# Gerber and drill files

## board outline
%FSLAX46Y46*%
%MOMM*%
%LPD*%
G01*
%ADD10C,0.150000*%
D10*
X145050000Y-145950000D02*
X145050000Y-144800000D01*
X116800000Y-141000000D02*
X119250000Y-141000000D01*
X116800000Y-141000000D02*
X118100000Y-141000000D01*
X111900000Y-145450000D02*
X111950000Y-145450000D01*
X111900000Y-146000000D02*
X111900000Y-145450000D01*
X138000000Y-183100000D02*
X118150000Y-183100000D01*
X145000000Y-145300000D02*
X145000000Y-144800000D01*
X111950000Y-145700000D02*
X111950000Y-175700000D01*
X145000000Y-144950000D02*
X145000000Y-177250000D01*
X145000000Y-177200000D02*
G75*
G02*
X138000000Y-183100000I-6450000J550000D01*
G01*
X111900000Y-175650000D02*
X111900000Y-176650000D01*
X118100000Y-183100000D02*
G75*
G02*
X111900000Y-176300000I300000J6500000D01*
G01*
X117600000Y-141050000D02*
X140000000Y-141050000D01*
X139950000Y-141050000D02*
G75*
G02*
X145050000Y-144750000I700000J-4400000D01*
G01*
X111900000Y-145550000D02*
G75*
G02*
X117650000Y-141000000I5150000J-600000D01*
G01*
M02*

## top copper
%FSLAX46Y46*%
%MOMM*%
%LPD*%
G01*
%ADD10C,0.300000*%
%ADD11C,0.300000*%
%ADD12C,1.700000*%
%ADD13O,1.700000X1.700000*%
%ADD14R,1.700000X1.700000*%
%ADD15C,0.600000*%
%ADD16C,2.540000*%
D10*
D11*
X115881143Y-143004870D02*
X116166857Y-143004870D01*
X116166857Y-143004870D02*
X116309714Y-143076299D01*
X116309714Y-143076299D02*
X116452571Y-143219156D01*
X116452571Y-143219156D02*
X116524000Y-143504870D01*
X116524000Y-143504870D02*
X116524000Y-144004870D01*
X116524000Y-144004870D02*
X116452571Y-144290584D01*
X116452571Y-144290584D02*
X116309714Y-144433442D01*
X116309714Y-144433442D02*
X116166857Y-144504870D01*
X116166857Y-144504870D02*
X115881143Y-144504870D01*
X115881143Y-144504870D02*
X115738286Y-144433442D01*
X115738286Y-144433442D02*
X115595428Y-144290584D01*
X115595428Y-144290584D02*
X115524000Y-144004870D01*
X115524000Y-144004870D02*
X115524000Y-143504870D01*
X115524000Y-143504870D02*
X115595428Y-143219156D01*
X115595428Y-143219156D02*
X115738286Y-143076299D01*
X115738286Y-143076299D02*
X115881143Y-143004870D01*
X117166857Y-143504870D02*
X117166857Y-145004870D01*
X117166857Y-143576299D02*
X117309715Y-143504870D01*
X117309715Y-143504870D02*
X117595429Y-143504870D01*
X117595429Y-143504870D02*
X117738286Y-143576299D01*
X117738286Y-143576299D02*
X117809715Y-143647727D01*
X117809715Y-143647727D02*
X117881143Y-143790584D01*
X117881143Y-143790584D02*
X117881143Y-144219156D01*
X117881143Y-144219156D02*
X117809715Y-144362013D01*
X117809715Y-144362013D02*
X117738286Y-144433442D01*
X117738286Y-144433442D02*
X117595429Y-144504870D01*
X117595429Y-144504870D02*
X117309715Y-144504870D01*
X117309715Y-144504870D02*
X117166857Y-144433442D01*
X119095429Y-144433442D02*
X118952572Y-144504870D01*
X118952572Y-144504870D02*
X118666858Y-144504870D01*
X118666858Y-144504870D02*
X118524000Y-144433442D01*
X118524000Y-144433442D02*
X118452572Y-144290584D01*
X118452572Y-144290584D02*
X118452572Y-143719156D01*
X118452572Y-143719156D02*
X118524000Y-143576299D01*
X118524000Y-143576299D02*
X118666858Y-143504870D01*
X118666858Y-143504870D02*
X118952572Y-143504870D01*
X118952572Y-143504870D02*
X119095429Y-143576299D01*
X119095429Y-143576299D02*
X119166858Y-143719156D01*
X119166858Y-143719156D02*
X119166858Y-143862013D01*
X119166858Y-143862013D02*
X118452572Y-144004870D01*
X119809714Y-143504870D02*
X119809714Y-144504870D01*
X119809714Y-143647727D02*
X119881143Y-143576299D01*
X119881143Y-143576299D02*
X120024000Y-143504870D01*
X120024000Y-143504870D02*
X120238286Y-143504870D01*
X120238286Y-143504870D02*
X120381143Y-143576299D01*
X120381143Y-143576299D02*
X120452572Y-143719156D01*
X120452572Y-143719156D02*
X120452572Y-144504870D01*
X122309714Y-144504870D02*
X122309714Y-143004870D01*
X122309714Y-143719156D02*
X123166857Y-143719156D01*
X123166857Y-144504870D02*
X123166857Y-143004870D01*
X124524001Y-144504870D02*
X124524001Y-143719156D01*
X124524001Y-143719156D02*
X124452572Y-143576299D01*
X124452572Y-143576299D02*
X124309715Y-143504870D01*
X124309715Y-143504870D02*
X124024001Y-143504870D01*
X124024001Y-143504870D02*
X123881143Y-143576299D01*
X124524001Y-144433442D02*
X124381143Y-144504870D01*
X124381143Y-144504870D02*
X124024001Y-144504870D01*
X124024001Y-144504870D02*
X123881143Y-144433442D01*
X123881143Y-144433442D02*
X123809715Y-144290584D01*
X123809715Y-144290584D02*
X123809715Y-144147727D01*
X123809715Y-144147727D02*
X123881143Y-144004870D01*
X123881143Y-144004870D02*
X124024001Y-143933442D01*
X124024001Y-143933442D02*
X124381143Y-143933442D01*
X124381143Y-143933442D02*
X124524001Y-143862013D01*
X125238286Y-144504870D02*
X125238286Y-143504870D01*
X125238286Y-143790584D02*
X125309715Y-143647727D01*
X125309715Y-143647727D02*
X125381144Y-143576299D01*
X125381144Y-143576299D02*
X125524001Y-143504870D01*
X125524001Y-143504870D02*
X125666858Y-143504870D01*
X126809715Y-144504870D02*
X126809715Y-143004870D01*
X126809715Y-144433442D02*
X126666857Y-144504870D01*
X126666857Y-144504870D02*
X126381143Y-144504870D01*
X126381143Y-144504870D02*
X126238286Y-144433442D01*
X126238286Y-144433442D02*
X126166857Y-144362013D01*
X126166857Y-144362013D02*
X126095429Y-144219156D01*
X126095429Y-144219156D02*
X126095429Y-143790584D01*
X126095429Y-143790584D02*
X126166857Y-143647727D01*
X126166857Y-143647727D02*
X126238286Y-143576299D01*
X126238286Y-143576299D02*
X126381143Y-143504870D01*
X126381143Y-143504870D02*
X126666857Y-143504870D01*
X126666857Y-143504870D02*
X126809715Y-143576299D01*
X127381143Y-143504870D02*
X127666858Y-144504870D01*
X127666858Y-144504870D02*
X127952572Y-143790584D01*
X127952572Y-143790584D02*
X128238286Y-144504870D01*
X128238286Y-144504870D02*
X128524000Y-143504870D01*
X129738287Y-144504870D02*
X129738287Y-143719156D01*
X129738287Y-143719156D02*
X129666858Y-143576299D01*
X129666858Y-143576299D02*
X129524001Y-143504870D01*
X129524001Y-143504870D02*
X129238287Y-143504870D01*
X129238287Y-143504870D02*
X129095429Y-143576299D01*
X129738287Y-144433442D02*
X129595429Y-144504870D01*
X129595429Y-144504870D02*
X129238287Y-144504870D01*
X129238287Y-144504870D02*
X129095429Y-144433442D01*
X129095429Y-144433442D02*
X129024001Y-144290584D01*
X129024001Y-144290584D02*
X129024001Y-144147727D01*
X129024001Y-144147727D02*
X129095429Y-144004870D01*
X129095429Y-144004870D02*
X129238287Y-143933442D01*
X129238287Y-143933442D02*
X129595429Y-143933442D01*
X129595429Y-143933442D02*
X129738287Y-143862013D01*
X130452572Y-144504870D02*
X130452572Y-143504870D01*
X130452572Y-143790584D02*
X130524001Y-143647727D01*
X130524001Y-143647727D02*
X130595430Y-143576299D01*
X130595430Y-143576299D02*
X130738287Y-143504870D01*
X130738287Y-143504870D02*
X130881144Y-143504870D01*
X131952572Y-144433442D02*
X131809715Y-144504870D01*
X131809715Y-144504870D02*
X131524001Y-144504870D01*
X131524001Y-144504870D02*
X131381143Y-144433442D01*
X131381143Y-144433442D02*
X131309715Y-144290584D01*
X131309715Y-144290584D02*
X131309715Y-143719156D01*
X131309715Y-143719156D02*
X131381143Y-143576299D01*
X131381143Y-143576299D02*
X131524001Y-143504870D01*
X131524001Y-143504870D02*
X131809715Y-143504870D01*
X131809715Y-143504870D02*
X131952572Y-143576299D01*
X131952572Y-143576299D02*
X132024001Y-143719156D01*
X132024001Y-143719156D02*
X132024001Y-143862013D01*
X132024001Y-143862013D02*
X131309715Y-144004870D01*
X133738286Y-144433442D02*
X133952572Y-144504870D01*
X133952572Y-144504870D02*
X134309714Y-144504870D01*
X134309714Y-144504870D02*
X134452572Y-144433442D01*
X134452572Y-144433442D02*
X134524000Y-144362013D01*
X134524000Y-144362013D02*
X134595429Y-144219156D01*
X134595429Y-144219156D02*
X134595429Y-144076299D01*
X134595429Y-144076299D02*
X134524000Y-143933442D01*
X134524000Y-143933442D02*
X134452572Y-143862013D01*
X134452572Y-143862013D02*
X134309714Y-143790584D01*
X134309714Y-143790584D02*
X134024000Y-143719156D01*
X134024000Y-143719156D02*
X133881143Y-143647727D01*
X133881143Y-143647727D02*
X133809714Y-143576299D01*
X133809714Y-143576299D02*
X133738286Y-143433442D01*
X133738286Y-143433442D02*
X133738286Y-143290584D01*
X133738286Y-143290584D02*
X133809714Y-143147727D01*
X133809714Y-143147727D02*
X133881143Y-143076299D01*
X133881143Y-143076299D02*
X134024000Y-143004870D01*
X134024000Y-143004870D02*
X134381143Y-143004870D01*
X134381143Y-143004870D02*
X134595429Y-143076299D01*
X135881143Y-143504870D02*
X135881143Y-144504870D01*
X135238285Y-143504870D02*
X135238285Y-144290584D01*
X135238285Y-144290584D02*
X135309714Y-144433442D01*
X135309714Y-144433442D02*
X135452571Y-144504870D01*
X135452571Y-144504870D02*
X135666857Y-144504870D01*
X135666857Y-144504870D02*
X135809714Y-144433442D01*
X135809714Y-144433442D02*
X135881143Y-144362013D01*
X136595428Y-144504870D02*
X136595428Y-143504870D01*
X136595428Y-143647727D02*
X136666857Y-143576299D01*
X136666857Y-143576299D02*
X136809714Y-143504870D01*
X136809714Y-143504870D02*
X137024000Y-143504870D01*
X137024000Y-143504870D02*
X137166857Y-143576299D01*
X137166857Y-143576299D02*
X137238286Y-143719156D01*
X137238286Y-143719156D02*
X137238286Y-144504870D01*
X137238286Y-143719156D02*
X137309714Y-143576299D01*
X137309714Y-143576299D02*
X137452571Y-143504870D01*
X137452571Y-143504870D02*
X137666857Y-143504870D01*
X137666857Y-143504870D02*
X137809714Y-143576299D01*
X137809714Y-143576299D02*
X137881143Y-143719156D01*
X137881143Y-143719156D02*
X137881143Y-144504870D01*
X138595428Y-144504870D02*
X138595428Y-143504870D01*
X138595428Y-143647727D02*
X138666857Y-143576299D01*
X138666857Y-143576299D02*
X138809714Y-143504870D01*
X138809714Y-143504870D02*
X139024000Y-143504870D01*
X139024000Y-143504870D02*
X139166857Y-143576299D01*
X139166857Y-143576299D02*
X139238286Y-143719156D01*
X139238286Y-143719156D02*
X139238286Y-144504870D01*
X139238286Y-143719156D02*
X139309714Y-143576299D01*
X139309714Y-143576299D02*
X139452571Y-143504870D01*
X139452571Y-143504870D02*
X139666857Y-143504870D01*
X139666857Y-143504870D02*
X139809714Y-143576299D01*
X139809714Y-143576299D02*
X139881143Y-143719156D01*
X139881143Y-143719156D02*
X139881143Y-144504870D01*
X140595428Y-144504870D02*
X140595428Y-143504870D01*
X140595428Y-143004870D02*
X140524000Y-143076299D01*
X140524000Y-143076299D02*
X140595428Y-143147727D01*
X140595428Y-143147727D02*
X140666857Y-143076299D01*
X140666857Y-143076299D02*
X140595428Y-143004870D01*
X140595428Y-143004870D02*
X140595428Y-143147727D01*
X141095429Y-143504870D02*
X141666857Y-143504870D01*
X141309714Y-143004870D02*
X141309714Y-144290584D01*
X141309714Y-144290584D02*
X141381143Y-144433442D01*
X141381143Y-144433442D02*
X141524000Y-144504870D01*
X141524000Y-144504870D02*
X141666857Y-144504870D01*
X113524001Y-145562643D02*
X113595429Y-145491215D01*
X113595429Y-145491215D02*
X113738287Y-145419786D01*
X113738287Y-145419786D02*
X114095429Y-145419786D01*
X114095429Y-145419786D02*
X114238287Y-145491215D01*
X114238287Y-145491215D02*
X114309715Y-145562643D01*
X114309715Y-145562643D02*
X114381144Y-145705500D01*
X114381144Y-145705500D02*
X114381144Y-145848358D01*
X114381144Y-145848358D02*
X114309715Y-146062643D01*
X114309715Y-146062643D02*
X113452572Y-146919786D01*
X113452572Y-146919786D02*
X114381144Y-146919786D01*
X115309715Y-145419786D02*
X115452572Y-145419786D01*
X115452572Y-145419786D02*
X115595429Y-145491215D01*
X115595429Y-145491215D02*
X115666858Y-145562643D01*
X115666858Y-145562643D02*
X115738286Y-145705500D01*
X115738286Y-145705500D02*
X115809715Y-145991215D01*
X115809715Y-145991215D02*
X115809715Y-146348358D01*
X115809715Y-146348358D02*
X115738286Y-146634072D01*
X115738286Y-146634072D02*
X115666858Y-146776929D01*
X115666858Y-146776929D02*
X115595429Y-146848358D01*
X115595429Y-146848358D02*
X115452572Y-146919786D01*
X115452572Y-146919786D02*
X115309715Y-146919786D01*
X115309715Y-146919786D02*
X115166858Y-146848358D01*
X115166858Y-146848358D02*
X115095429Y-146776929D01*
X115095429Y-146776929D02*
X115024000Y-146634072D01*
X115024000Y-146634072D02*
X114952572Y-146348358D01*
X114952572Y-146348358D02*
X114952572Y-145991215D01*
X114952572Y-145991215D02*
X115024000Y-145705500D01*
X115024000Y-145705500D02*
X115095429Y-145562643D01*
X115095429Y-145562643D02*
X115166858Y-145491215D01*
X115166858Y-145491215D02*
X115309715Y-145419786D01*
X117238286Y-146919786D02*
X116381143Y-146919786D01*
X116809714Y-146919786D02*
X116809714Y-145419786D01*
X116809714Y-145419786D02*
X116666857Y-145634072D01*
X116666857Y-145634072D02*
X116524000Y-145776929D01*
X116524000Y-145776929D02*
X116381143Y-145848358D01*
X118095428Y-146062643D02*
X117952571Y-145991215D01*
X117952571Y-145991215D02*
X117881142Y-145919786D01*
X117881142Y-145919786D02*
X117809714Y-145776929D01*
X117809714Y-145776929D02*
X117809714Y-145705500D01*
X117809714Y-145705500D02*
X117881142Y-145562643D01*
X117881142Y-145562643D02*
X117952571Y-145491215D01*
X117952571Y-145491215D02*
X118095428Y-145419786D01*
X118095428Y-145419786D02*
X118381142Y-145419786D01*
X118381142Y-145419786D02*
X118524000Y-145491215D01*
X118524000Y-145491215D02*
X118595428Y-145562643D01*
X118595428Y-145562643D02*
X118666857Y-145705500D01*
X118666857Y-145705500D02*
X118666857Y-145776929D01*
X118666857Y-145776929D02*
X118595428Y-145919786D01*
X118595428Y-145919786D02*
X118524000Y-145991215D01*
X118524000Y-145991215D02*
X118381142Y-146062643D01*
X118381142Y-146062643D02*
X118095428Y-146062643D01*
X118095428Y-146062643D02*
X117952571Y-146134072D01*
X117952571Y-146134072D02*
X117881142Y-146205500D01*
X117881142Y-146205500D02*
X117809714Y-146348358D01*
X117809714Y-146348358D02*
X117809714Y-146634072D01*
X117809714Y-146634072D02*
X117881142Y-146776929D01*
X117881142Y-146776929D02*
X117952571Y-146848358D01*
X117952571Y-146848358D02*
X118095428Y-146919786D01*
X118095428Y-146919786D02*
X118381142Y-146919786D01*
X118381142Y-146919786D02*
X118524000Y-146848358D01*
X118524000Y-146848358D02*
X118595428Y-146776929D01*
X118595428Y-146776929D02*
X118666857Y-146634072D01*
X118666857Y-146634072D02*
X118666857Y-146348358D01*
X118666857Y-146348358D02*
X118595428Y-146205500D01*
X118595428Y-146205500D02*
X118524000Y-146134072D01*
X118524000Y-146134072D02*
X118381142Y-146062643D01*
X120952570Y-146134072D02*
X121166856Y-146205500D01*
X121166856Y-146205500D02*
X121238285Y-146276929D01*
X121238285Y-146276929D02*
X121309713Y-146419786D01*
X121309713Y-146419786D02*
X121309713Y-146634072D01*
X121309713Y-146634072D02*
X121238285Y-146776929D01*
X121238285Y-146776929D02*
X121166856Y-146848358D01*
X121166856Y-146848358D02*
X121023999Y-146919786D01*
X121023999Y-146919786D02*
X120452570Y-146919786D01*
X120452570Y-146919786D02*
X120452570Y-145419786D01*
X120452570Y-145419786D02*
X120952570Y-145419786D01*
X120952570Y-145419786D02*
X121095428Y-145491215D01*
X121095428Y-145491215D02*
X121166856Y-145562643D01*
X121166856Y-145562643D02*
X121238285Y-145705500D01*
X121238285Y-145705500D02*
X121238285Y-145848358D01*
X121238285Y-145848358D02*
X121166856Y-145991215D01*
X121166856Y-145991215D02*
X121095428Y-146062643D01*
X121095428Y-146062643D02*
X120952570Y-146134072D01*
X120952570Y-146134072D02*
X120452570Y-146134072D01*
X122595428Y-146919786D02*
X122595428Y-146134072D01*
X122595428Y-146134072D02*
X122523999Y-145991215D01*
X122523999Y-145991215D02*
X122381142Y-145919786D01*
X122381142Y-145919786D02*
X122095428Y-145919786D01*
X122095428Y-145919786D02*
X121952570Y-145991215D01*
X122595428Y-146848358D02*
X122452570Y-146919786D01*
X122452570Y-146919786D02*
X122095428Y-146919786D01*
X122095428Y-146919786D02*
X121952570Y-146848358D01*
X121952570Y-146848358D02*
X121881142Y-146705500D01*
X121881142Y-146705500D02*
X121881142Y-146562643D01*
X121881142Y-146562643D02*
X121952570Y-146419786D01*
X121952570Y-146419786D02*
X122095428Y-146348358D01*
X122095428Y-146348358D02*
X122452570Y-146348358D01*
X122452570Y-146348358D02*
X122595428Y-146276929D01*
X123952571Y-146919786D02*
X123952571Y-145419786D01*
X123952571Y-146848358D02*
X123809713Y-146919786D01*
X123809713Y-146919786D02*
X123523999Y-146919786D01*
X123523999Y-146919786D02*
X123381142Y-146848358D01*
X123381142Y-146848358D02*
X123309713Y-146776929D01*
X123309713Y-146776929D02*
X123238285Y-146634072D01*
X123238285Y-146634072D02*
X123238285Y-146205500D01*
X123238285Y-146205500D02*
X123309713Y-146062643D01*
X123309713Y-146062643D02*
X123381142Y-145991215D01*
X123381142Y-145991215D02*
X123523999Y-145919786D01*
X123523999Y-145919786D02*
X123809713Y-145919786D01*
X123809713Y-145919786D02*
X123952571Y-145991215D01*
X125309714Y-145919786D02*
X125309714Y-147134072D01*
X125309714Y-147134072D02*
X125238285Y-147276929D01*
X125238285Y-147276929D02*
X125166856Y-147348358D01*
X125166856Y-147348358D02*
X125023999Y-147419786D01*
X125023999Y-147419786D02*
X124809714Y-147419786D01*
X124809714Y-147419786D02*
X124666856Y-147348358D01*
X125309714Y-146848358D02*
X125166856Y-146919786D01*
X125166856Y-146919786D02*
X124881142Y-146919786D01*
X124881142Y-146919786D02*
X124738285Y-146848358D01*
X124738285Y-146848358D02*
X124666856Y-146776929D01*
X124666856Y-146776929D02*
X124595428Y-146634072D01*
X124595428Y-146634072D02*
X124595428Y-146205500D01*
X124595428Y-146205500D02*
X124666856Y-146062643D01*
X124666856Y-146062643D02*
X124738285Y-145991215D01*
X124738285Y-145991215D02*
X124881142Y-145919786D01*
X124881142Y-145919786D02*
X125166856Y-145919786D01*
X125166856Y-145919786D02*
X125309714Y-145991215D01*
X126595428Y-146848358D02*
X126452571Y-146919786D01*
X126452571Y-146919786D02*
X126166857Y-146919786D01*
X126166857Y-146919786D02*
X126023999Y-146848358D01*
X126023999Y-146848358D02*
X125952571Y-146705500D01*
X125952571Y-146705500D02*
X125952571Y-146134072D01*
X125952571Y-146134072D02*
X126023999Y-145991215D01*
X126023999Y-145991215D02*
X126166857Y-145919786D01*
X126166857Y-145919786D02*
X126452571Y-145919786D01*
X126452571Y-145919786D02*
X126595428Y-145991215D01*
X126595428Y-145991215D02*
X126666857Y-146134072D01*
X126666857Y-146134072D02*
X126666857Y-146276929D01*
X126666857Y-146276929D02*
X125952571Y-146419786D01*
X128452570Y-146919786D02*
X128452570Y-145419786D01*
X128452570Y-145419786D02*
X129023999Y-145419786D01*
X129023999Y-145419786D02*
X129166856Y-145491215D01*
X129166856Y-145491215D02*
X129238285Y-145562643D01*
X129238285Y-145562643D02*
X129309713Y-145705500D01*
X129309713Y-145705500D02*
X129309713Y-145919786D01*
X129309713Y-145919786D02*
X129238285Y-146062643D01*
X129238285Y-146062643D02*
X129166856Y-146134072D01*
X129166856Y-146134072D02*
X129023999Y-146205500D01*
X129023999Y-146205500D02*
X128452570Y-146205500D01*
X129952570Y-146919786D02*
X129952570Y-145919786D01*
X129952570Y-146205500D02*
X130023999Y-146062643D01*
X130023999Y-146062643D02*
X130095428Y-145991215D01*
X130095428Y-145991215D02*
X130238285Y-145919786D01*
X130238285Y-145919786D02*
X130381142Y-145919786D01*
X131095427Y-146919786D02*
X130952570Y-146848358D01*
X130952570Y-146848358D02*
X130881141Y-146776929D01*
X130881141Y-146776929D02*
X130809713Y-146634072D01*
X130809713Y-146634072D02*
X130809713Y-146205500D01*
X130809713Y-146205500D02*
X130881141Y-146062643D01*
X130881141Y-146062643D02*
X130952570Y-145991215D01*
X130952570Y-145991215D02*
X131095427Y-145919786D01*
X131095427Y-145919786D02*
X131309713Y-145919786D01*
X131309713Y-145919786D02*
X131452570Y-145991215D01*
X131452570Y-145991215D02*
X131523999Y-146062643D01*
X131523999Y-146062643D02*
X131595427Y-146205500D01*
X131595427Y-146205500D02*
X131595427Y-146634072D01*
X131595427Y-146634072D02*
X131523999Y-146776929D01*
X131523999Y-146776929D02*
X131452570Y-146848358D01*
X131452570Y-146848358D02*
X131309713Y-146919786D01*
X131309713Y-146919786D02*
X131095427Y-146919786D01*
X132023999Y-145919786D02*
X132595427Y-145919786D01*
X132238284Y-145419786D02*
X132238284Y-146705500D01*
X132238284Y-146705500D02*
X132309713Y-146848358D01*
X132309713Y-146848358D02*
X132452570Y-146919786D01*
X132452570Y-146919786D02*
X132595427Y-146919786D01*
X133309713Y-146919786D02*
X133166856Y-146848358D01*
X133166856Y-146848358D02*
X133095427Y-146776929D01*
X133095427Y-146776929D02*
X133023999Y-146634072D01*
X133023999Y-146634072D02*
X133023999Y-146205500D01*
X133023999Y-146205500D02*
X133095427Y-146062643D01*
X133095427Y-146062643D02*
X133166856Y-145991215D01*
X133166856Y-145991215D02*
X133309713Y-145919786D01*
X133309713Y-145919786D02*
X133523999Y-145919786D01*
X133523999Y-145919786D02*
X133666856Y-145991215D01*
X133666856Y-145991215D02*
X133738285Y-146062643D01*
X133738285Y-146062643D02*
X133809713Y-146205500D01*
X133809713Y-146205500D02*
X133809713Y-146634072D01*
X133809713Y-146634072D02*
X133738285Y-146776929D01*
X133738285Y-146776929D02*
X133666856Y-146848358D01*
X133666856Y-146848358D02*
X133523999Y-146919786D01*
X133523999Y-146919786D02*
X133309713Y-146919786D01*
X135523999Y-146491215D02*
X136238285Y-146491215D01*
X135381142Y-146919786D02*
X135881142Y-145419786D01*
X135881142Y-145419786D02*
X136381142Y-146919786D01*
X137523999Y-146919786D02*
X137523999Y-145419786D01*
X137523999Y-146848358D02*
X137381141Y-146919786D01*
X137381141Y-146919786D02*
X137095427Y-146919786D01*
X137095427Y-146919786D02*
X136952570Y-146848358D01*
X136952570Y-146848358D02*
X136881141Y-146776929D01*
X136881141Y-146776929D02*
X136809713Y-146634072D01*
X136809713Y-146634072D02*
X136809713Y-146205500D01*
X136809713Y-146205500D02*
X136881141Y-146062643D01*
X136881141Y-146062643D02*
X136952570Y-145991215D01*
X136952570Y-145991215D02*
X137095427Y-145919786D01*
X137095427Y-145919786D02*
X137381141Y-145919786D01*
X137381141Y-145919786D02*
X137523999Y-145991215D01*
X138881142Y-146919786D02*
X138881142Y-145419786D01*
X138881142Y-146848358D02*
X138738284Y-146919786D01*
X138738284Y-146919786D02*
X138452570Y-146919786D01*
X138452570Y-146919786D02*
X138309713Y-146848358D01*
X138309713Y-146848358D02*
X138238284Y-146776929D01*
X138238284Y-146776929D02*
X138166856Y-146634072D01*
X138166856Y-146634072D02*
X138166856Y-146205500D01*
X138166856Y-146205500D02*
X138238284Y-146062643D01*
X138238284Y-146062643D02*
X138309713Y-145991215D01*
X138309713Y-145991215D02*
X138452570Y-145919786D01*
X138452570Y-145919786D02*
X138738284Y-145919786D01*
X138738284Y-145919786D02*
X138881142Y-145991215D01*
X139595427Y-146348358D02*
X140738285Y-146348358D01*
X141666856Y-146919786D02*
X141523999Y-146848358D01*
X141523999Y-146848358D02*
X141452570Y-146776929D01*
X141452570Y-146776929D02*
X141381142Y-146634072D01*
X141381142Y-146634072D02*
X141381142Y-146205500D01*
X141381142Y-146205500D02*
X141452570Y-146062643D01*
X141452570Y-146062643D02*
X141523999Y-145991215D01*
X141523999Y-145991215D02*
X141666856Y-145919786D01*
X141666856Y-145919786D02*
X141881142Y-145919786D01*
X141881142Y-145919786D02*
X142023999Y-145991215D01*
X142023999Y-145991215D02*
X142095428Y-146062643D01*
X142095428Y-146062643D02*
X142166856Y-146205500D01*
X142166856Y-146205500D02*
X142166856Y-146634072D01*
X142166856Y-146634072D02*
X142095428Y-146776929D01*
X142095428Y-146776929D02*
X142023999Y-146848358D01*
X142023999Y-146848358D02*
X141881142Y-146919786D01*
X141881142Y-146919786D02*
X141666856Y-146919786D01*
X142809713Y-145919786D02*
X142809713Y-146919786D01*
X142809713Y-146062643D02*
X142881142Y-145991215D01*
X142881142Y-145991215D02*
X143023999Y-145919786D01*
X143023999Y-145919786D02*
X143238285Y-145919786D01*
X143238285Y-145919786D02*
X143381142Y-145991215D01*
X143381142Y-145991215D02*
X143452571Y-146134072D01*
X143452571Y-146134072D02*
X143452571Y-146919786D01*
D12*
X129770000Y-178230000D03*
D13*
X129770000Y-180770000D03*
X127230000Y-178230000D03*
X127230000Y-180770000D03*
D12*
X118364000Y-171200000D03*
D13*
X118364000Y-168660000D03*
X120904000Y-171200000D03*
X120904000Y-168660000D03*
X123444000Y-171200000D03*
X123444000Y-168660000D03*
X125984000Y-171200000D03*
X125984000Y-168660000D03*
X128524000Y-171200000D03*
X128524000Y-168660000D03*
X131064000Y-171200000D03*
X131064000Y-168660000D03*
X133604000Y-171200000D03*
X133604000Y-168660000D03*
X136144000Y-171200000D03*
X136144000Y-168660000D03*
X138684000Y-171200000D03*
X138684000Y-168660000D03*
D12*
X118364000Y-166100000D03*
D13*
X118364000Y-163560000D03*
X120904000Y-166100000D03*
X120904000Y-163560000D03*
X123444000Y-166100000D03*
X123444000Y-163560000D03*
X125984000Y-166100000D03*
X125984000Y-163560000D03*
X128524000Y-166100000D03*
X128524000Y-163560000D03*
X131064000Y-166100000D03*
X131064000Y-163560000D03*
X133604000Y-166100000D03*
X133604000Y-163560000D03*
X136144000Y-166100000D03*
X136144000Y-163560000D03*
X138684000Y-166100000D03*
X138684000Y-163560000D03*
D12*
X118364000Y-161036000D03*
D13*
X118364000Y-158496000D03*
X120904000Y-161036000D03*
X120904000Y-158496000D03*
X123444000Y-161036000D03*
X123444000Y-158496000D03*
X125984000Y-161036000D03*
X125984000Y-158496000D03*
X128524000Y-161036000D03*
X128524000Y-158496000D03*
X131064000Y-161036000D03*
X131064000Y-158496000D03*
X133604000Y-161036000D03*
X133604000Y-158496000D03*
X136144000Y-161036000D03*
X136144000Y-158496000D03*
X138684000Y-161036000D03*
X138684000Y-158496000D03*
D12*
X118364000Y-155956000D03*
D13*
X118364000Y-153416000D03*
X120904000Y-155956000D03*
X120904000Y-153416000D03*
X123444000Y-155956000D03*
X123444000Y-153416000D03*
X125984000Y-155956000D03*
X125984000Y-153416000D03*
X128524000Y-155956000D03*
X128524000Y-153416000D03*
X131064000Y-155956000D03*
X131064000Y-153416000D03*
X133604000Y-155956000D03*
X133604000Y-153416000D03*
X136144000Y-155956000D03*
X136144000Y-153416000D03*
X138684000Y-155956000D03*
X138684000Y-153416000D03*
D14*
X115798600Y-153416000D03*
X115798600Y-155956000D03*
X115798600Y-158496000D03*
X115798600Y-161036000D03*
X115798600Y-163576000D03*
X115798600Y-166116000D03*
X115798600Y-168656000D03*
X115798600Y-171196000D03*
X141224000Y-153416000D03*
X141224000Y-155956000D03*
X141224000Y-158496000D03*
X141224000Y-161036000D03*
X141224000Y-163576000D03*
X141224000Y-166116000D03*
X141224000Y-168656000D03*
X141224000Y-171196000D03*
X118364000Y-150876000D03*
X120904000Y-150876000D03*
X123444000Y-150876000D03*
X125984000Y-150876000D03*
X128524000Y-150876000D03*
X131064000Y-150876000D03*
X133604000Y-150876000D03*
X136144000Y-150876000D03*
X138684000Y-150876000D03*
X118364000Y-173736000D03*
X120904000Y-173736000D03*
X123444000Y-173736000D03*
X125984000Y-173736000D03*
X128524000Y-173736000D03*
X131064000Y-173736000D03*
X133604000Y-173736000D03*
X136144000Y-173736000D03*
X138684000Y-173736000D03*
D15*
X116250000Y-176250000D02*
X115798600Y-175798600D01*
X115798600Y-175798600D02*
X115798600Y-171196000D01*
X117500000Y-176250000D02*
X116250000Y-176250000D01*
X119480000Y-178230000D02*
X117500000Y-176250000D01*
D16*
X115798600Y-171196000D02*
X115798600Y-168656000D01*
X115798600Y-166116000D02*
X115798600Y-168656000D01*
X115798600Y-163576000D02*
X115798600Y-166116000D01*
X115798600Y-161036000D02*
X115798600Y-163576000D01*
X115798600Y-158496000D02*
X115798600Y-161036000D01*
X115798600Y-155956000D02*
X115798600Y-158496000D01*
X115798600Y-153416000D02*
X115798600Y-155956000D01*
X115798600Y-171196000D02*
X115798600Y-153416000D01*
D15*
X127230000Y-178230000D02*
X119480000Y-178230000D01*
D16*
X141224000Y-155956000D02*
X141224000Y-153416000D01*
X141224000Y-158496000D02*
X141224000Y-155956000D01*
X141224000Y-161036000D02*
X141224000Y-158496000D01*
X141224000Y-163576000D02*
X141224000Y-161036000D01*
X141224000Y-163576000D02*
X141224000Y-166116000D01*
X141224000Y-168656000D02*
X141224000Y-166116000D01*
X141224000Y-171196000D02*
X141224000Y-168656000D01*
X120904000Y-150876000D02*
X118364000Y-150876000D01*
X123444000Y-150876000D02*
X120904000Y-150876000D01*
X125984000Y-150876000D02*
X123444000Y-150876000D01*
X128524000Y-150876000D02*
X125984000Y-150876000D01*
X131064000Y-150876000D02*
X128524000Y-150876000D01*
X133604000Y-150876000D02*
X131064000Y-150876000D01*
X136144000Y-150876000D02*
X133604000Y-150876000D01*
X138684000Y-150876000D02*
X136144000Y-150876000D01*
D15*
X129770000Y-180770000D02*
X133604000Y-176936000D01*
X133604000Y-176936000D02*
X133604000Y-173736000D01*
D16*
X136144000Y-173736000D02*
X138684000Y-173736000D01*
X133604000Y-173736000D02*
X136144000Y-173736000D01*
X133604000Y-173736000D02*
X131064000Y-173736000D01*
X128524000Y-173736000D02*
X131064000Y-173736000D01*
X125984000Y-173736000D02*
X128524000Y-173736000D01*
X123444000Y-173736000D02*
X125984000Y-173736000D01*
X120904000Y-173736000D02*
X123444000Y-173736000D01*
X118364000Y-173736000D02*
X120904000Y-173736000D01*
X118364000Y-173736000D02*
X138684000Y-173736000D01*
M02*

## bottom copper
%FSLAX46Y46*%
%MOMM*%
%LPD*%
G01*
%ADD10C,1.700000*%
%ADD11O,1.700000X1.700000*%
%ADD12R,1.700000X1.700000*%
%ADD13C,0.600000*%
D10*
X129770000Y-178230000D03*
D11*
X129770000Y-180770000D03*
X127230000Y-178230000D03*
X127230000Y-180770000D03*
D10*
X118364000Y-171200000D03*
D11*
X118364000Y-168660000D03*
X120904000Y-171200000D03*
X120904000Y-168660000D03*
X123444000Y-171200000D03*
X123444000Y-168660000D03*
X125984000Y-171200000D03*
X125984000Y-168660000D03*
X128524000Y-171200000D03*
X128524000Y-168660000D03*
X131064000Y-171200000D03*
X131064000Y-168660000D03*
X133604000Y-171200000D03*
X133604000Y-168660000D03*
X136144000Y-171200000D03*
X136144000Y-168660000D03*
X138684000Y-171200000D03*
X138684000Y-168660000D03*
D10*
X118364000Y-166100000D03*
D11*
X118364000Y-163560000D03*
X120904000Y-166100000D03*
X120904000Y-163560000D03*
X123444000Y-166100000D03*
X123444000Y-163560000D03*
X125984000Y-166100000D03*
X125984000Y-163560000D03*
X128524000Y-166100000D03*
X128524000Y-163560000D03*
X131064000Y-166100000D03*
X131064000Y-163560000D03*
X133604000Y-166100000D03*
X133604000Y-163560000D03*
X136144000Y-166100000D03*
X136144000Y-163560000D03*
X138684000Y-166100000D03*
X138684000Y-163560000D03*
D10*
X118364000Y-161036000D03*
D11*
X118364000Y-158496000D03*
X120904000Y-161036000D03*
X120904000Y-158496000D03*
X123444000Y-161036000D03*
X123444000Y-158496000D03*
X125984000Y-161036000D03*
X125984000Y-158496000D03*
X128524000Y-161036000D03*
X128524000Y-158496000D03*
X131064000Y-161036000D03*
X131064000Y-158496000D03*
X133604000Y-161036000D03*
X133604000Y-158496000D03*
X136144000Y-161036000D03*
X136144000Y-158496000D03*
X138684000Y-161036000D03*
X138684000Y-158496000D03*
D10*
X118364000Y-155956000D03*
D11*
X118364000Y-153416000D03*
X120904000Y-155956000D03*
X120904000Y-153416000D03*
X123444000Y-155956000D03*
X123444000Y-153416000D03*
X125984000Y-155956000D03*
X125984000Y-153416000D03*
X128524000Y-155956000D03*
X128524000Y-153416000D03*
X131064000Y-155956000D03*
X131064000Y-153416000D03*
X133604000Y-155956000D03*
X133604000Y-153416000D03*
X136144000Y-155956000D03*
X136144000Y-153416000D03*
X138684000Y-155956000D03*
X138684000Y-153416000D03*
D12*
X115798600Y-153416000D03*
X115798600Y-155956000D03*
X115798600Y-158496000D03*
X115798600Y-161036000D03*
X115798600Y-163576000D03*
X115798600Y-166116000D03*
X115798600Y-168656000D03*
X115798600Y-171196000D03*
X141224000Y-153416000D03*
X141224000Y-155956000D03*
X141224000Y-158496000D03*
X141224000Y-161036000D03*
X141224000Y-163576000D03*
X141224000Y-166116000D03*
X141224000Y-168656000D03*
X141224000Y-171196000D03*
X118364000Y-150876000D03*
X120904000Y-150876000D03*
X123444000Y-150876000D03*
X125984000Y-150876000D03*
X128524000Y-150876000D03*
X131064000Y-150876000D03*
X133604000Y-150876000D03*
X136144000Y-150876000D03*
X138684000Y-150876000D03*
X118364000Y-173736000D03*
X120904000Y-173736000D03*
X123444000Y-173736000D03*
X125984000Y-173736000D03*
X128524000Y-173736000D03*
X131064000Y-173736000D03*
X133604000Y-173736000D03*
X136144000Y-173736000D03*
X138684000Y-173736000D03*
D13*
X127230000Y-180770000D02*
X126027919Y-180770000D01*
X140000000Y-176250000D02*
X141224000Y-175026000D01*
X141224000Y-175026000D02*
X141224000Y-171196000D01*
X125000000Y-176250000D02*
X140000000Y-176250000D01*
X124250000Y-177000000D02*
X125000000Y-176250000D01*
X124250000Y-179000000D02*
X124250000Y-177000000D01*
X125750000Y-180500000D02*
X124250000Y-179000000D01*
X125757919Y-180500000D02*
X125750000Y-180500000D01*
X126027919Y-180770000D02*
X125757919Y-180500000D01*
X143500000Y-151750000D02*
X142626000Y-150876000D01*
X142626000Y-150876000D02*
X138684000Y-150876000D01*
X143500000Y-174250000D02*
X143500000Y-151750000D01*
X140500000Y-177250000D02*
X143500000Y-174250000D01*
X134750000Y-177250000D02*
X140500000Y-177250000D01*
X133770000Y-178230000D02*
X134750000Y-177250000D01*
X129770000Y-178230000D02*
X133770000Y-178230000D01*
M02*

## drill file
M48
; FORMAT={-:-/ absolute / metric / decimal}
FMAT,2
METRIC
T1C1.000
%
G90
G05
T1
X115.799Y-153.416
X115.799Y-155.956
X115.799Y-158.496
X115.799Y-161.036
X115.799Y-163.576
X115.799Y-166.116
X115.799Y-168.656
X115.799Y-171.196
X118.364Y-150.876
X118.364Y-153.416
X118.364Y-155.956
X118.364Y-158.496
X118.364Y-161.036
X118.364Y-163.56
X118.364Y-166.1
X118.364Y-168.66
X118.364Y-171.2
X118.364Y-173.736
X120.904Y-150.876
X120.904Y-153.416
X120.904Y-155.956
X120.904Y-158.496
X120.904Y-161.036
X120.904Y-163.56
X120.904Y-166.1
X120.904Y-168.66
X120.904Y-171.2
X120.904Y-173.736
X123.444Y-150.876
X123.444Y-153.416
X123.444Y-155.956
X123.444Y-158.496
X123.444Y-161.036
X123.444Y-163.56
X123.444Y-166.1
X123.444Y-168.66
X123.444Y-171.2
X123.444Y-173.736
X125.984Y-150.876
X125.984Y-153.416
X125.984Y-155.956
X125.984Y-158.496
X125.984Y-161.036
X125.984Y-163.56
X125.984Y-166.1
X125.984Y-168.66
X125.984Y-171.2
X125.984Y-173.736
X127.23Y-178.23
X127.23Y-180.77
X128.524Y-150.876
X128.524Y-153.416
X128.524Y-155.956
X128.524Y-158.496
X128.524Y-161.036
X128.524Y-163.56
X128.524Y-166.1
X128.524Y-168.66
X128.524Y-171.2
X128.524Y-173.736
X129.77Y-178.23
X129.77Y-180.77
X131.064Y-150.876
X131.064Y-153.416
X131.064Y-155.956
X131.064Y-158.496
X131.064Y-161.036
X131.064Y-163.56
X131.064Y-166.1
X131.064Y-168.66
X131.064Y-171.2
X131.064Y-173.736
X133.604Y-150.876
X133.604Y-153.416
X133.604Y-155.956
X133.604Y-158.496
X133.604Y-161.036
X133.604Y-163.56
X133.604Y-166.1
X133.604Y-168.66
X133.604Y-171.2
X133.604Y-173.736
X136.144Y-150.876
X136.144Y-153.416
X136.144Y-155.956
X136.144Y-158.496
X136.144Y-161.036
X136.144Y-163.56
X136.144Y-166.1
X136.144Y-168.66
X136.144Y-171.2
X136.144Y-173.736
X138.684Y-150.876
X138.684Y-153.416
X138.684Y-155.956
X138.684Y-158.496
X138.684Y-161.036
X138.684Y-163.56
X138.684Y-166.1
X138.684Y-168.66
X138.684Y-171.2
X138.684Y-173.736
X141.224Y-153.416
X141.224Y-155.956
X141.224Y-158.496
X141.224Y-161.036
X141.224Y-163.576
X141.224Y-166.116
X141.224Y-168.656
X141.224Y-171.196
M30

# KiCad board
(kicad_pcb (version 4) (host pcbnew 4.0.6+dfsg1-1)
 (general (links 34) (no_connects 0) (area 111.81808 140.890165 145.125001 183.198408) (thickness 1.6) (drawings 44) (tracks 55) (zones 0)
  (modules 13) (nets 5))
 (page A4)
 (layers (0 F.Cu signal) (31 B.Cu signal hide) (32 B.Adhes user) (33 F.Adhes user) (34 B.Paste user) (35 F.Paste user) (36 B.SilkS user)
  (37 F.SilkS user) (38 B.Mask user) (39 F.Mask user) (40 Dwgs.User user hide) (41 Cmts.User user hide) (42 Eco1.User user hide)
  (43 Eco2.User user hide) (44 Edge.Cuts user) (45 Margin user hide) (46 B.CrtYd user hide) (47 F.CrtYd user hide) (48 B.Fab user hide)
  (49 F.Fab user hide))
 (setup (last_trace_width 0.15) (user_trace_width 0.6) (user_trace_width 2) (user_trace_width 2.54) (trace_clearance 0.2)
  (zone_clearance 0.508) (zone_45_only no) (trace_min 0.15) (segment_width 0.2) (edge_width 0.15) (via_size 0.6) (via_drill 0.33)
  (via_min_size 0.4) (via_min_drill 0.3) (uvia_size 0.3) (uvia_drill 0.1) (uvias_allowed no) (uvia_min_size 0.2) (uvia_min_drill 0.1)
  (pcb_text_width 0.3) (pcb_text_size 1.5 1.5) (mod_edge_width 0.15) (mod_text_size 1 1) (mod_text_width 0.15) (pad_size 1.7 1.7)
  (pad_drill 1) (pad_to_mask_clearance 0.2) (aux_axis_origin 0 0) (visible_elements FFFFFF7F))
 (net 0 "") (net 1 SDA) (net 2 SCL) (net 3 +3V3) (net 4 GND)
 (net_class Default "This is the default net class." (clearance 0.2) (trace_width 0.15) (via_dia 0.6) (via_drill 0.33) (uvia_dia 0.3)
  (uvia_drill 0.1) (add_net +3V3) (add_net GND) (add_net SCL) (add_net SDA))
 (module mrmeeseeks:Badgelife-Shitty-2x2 (layer F.Cu) (at 128.5 179.5)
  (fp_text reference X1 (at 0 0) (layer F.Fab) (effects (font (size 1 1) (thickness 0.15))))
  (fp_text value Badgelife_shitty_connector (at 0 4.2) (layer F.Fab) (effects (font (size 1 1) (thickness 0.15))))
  (pad 4 thru_hole circle (at 1.27 -1.27) (size 1.7 1.7) (drill 1) (layers *.Cu *.Mask) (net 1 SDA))
  (pad 3 thru_hole oval (at 1.27 1.27) (size 1.7 1.7) (drill 1) (layers *.Cu *.Mask) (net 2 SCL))
  (pad 1 thru_hole oval (at -1.27 -1.27) (size 1.7 1.7) (drill 1) (layers *.Cu *.Mask) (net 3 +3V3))
  (pad 2 thru_hole oval (at -1.27 1.27) (size 1.7 1.7) (drill 1) (layers *.Cu *.Mask) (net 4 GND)))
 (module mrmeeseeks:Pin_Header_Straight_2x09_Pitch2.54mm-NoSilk (layer F.Cu) (at 118.364 171.2 90)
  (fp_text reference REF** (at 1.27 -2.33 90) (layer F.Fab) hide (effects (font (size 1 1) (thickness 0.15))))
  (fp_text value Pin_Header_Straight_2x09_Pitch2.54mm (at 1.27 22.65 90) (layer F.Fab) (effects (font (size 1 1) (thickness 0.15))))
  (pad 1 thru_hole circle (at 0 0 90) (size 1.7 1.7) (drill 1) (layers *.Cu *.Mask))
  (pad 2 thru_hole oval (at 2.54 0 90) (size 1.7 1.7) (drill 1) (layers *.Cu *.Mask))
  (pad 3 thru_hole oval (at 0 2.54 90) (size 1.7 1.7) (drill 1) (layers *.Cu *.Mask))
  (pad 4 thru_hole oval (at 2.54 2.54 90) (size 1.7 1.7) (drill 1) (layers *.Cu *.Mask))
  (pad 5 thru_hole oval (at 0 5.08 90) (size 1.7 1.7) (drill 1) (layers *.Cu *.Mask))
  (pad 6 thru_hole oval (at 2.54 5.08 90) (size 1.7 1.7) (drill 1) (layers *.Cu *.Mask))
  (pad 7 thru_hole oval (at 0 7.62 90) (size 1.7 1.7) (drill 1) (layers *.Cu *.Mask))
  (pad 8 thru_hole oval (at 2.54 7.62 90) (size 1.7 1.7) (drill 1) (layers *.Cu *.Mask))
  (pad 9 thru_hole oval (at 0 10.16 90) (size 1.7 1.7) (drill 1) (layers *.Cu *.Mask))
  (pad 10 thru_hole oval (at 2.54 10.16 90) (size 1.7 1.7) (drill 1) (layers *.Cu *.Mask))
  (pad 11 thru_hole oval (at 0 12.7 90) (size 1.7 1.7) (drill 1) (layers *.Cu *.Mask))
  (pad 12 thru_hole oval (at 2.54 12.7 90) (size 1.7 1.7) (drill 1) (layers *.Cu *.Mask))
  (pad 13 thru_hole oval (at 0 15.24 90) (size 1.7 1.7) (drill 1) (layers *.Cu *.Mask))
  (pad 14 thru_hole oval (at 2.54 15.24 90) (size 1.7 1.7) (drill 1) (layers *.Cu *.Mask))
  (pad 15 thru_hole oval (at 0 17.78 90) (size 1.7 1.7) (drill 1) (layers *.Cu *.Mask))
  (pad 16 thru_hole oval (at 2.54 17.78 90) (size 1.7 1.7) (drill 1) (layers *.Cu *.Mask))
  (pad 17 thru_hole oval (at 0 20.32 90) (size 1.7 1.7) (drill 1) (layers *.Cu *.Mask))
  (pad 18 thru_hole oval (at 2.54 20.32 90) (size 1.7 1.7) (drill 1) (layers *.Cu *.Mask)))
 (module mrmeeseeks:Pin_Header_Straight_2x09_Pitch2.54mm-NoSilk (layer F.Cu) (at 118.364 166.1 90)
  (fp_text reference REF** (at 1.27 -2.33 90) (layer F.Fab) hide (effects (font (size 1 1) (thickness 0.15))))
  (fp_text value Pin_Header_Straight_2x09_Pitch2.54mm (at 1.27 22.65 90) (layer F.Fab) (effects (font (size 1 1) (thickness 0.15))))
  (pad 1 thru_hole circle (at 0 0 90) (size 1.7 1.7) (drill 1) (layers *.Cu *.Mask))
  (pad 2 thru_hole oval (at 2.54 0 90) (size 1.7 1.7) (drill 1) (layers *.Cu *.Mask))
  (pad 3 thru_hole oval (at 0 2.54 90) (size 1.7 1.7) (drill 1) (layers *.Cu *.Mask))
  (pad 4 thru_hole oval (at 2.54 2.54 90) (size 1.7 1.7) (drill 1) (layers *.Cu *.Mask))
  (pad 5 thru_hole oval (at 0 5.08 90) (size 1.7 1.7) (drill 1) (layers *.Cu *.Mask))
  (pad 6 thru_hole oval (at 2.54 5.08 90) (size 1.7 1.7) (drill 1) (layers *.Cu *.Mask))
  (pad 7 thru_hole oval (at 0 7.62 90) (size 1.7 1.7) (drill 1) (layers *.Cu *.Mask))
  (pad 8 thru_hole oval (at 2.54 7.62 90) (size 1.7 1.7) (drill 1) (layers *.Cu *.Mask))
  (pad 9 thru_hole oval (at 0 10.16 90) (size 1.7 1.7) (drill 1) (layers *.Cu *.Mask))
  (pad 10 thru_hole oval (at 2.54 10.16 90) (size 1.7 1.7) (drill 1) (layers *.Cu *.Mask))
  (pad 11 thru_hole oval (at 0 12.7 90) (size 1.7 1.7) (drill 1) (layers *.Cu *.Mask))
  (pad 12 thru_hole oval (at 2.54 12.7 90) (size 1.7 1.7) (drill 1) (layers *.Cu *.Mask))
  (pad 13 thru_hole oval (at 0 15.24 90) (size 1.7 1.7) (drill 1) (layers *.Cu *.Mask))
  (pad 14 thru_hole oval (at 2.54 15.24 90) (size 1.7 1.7) (drill 1) (layers *.Cu *.Mask))
  (pad 15 thru_hole oval (at 0 17.78 90) (size 1.7 1.7) (drill 1) (layers *.Cu *.Mask))
  (pad 16 thru_hole oval (at 2.54 17.78 90) (size 1.7 1.7) (drill 1) (layers *.Cu *.Mask))
  (pad 17 thru_hole oval (at 0 20.32 90) (size 1.7 1.7) (drill 1) (layers *.Cu *.Mask))
  (pad 18 thru_hole oval (at 2.54 20.32 90) (size 1.7 1.7) (drill 1) (layers *.Cu *.Mask)))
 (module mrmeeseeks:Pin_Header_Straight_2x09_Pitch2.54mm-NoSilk (layer F.Cu) (at 118.364 161.036 90)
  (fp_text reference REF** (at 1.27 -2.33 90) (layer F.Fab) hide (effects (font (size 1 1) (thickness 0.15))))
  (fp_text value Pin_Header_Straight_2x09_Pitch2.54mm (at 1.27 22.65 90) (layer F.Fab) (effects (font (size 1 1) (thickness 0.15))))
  (pad 1 thru_hole circle (at 0 0 90) (size 1.7 1.7) (drill 1) (layers *.Cu *.Mask))
  (pad 2 thru_hole oval (at 2.54 0 90) (size 1.7 1.7) (drill 1) (layers *.Cu *.Mask))
  (pad 3 thru_hole oval (at 0 2.54 90) (size 1.7 1.7) (drill 1) (layers *.Cu *.Mask))
  (pad 4 thru_hole oval (at 2.54 2.54 90) (size 1.7 1.7) (drill 1) (layers *.Cu *.Mask))
  (pad 5 thru_hole oval (at 0 5.08 90) (size 1.7 1.7) (drill 1) (layers *.Cu *.Mask))
  (pad 6 thru_hole oval (at 2.54 5.08 90) (size 1.7 1.7) (drill 1) (layers *.Cu *.Mask))
  (pad 7 thru_hole oval (at 0 7.62 90) (size 1.7 1.7) (drill 1) (layers *.Cu *.Mask))
  (pad 8 thru_hole oval (at 2.54 7.62 90) (size 1.7 1.7) (drill 1) (layers *.Cu *.Mask))
  (pad 9 thru_hole oval (at 0 10.16 90) (size 1.7 1.7) (drill 1) (layers *.Cu *.Mask))
  (pad 10 thru_hole oval (at 2.54 10.16 90) (size 1.7 1.7) (drill 1) (layers *.Cu *.Mask))
  (pad 11 thru_hole oval (at 0 12.7 90) (size 1.7 1.7) (drill 1) (layers *.Cu *.Mask))
  (pad 12 thru_hole oval (at 2.54 12.7 90) (size 1.7 1.7) (drill 1) (layers *.Cu *.Mask))
  (pad 13 thru_hole oval (at 0 15.24 90) (size 1.7 1.7) (drill 1) (layers *.Cu *.Mask))
  (pad 14 thru_hole oval (at 2.54 15.24 90) (size 1.7 1.7) (drill 1) (layers *.Cu *.Mask))
  (pad 15 thru_hole oval (at 0 17.78 90) (size 1.7 1.7) (drill 1) (layers *.Cu *.Mask))
  (pad 16 thru_hole oval (at 2.54 17.78 90) (size 1.7 1.7) (drill 1) (layers *.Cu *.Mask))
  (pad 17 thru_hole oval (at 0 20.32 90) (size 1.7 1.7) (drill 1) (layers *.Cu *.Mask))
  (pad 18 thru_hole oval (at 2.54 20.32 90) (size 1.7 1.7) (drill 1) (layers *.Cu *.Mask)))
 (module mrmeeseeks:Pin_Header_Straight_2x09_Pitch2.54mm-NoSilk (layer F.Cu) (at 118.364 155.956 90)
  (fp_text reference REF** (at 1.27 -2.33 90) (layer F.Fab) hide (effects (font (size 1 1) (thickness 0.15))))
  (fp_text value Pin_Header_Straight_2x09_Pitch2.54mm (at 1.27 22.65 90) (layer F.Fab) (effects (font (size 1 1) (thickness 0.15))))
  (pad 1 thru_hole circle (at 0 0 90) (size 1.7 1.7) (drill 1) (layers *.Cu *.Mask))
  (pad 2 thru_hole oval (at 2.54 0 90) (size 1.7 1.7) (drill 1) (layers *.Cu *.Mask))
  (pad 3 thru_hole oval (at 0 2.54 90) (size 1.7 1.7) (drill 1) (layers *.Cu *.Mask))
  (pad 4 thru_hole oval (at 2.54 2.54 90) (size 1.7 1.7) (drill 1) (layers *.Cu *.Mask))
  (pad 5 thru_hole oval (at 0 5.08 90) (size 1.7 1.7) (drill 1) (layers *.Cu *.Mask))
  (pad 6 thru_hole oval (at 2.54 5.08 90) (size 1.7 1.7) (drill 1) (layers *.Cu *.Mask))
  (pad 7 thru_hole oval (at 0 7.62 90) (size 1.7 1.7) (drill 1) (layers *.Cu *.Mask))
  (pad 8 thru_hole oval (at 2.54 7.62 90) (size 1.7 1.7) (drill 1) (layers *.Cu *.Mask))
  (pad 9 thru_hole oval (at 0 10.16 90) (size 1.7 1.7) (drill 1) (layers *.Cu *.Mask))
  (pad 10 thru_hole oval (at 2.54 10.16 90) (size 1.7 1.7) (drill 1) (layers *.Cu *.Mask))
  (pad 11 thru_hole oval (at 0 12.7 90) (size 1.7 1.7) (drill 1) (layers *.Cu *.Mask))
  (pad 12 thru_hole oval (at 2.54 12.7 90) (size 1.7 1.7) (drill 1) (layers *.Cu *.Mask))
  (pad 13 thru_hole oval (at 0 15.24 90) (size 1.7 1.7) (drill 1) (layers *.Cu *.Mask))
  (pad 14 thru_hole oval (at 2.54 15.24 90) (size 1.7 1.7) (drill 1) (layers *.Cu *.Mask))
  (pad 15 thru_hole oval (at 0 17.78 90) (size 1.7 1.7) (drill 1) (layers *.Cu *.Mask))
  (pad 16 thru_hole oval (at 2.54 17.78 90) (size 1.7 1.7) (drill 1) (layers *.Cu *.Mask))
  (pad 17 thru_hole oval (at 0 20.32 90) (size 1.7 1.7) (drill 1) (layers *.Cu *.Mask))
  (pad 18 thru_hole oval (at 2.54 20.32 90) (size 1.7 1.7) (drill 1) (layers *.Cu *.Mask)))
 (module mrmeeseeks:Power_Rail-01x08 (layer F.Cu) (at 115.7986 153.416)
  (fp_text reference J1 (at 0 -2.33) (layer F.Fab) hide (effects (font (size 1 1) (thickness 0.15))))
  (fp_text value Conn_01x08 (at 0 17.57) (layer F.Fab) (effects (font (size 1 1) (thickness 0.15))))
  (pad 1 thru_hole rect (at 0 0) (size 1.7 1.7) (drill 1) (layers *.Cu *.Mask) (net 3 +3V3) (solder_mask_margin 0.1))
  (pad 2 thru_hole rect (at 0 2.54) (size 1.7 1.7) (drill 1) (layers *.Cu *.Mask) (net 3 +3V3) (solder_mask_margin 0.1))
  (pad 3 thru_hole rect (at 0 5.08) (size 1.7 1.7) (drill 1) (layers *.Cu *.Mask) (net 3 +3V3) (solder_mask_margin 0.1))
  (pad 4 thru_hole rect (at 0 7.62) (size 1.7 1.7) (drill 1) (layers *.Cu *.Mask) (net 3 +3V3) (solder_mask_margin 0.1))
  (pad 5 thru_hole rect (at 0 10.16) (size 1.7 1.7) (drill 1) (layers *.Cu *.Mask) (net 3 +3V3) (solder_mask_margin 0.1))
  (pad 6 thru_hole rect (at 0 12.7) (size 1.7 1.7) (drill 1) (layers *.Cu *.Mask) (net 3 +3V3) (solder_mask_margin 0.1))
  (pad 7 thru_hole rect (at 0 15.24) (size 1.7 1.7) (drill 1) (layers *.Cu *.Mask) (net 3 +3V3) (solder_mask_margin 0.1))
  (pad 8 thru_hole rect (at 0 17.78) (size 1.7 1.7) (drill 1) (layers *.Cu *.Mask) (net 3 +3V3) (solder_mask_margin 0.1)))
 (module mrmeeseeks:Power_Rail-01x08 (layer F.Cu) (at 141.224 153.416)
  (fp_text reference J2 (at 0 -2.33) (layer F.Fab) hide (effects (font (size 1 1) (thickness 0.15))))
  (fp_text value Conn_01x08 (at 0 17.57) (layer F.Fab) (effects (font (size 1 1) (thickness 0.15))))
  (pad 1 thru_hole rect (at 0 0) (size 1.7 1.7) (drill 1) (layers *.Cu *.Mask) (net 4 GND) (solder_mask_margin 0.1))
  (pad 2 thru_hole rect (at 0 2.54) (size 1.7 1.7) (drill 1) (layers *.Cu *.Mask) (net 4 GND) (solder_mask_margin 0.1))
  (pad 3 thru_hole rect (at 0 5.08) (size 1.7 1.7) (drill 1) (layers *.Cu *.Mask) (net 4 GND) (solder_mask_margin 0.1))
  (pad 4 thru_hole rect (at 0 7.62) (size 1.7 1.7) (drill 1) (layers *.Cu *.Mask) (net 4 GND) (solder_mask_margin 0.1))
  (pad 5 thru_hole rect (at 0 10.16) (size 1.7 1.7) (drill 1) (layers *.Cu *.Mask) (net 4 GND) (solder_mask_margin 0.1))
  (pad 6 thru_hole rect (at 0 12.7) (size 1.7 1.7) (drill 1) (layers *.Cu *.Mask) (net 4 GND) (solder_mask_margin 0.1))
  (pad 7 thru_hole rect (at 0 15.24) (size 1.7 1.7) (drill 1) (layers *.Cu *.Mask) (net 4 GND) (solder_mask_margin 0.1))
  (pad 8 thru_hole rect (at 0 17.78) (size 1.7 1.7) (drill 1) (layers *.Cu *.Mask) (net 4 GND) (solder_mask_margin 0.1)))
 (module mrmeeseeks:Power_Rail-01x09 (layer F.Cu) (at 118.364 150.876 90)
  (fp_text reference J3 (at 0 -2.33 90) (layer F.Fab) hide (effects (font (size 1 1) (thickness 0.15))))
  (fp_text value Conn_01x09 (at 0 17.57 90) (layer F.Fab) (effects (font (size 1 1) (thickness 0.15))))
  (pad 1 thru_hole rect (at 0 0 90) (size 1.7 1.7) (drill 1) (layers *.Cu *.Mask) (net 1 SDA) (solder_mask_margin 0.1))
  (pad 2 thru_hole rect (at 0 2.54 90) (size 1.7 1.7) (drill 1) (layers *.Cu *.Mask) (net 1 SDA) (solder_mask_margin 0.1))
  (pad 3 thru_hole rect (at 0 5.08 90) (size 1.7 1.7) (drill 1) (layers *.Cu *.Mask) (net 1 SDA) (solder_mask_margin 0.1))
  (pad 4 thru_hole rect (at 0 7.62 90) (size 1.7 1.7) (drill 1) (layers *.Cu *.Mask) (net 1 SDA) (solder_mask_margin 0.1))
  (pad 5 thru_hole rect (at 0 10.16 90) (size 1.7 1.7) (drill 1) (layers *.Cu *.Mask) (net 1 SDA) (solder_mask_margin 0.1))
  (pad 6 thru_hole rect (at 0 12.7 90) (size 1.7 1.7) (drill 1) (layers *.Cu *.Mask) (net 1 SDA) (solder_mask_margin 0.1))
  (pad 7 thru_hole rect (at 0 15.24 90) (size 1.7 1.7) (drill 1) (layers *.Cu *.Mask) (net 1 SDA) (solder_mask_margin 0.1))
  (pad 8 thru_hole rect (at 0 17.78 90) (size 1.7 1.7) (drill 1) (layers *.Cu *.Mask) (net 1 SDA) (solder_mask_margin 0.1))
  (pad 9 thru_hole rect (at 0 20.32 90) (size 1.7 1.7) (drill 1) (layers *.Cu *.Mask) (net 1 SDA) (solder_mask_margin 0.1)))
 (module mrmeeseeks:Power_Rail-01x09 (layer F.Cu) (at 118.364 173.736 90)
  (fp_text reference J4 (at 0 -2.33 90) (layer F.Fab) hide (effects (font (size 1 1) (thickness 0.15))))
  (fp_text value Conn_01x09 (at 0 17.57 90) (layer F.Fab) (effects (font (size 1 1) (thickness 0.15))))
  (pad 1 thru_hole rect (at 0 0 90) (size 1.7 1.7) (drill 1) (layers *.Cu *.Mask) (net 2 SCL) (solder_mask_margin 0.1))
  (pad 2 thru_hole rect (at 0 2.54 90) (size 1.7 1.7) (drill 1) (layers *.Cu *.Mask) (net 2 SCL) (solder_mask_margin 0.1))
  (pad 3 thru_hole rect (at 0 5.08 90) (size 1.7 1.7) (drill 1) (layers *.Cu *.Mask) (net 2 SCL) (solder_mask_margin 0.1))
  (pad 4 thru_hole rect (at 0 7.62 90) (size 1.7 1.7) (drill 1) (layers *.Cu *.Mask) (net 2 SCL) (solder_mask_margin 0.1))
  (pad 5 thru_hole rect (at 0 10.16 90) (size 1.7 1.7) (drill 1) (layers *.Cu *.Mask) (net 2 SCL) (solder_mask_margin 0.1))
  (pad 6 thru_hole rect (at 0 12.7 90) (size 1.7 1.7) (drill 1) (layers *.Cu *.Mask) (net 2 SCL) (solder_mask_margin 0.1))
  (pad 7 thru_hole rect (at 0 15.24 90) (size 1.7 1.7) (drill 1) (layers *.Cu *.Mask) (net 2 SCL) (solder_mask_margin 0.1))
  (pad 8 thru_hole rect (at 0 17.78 90) (size 1.7 1.7) (drill 1) (layers *.Cu *.Mask) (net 2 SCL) (solder_mask_margin 0.1))
  (pad 9 thru_hole rect (at 0 20.32 90) (size 1.7 1.7) (drill 1) (layers *.Cu *.Mask) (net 2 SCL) (solder_mask_margin 0.1)))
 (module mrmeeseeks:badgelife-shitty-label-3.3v (layer F.Cu) (at 113.4 162.2 90)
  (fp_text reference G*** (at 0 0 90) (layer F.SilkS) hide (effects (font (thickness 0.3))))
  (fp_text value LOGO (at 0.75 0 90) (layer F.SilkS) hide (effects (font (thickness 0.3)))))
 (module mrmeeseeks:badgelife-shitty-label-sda (layer F.Cu) (at 128.2 148.8)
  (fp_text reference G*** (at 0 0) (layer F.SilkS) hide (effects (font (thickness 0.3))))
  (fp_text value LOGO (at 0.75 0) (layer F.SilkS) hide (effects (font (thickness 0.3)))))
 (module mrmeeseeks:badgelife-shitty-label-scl (layer F.Cu) (at 128.4 175.7)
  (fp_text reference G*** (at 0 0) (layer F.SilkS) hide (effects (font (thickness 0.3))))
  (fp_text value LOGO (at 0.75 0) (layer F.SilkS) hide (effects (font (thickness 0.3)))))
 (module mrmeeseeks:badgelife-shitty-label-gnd (layer F.Cu) (at 143.7 162.3 270)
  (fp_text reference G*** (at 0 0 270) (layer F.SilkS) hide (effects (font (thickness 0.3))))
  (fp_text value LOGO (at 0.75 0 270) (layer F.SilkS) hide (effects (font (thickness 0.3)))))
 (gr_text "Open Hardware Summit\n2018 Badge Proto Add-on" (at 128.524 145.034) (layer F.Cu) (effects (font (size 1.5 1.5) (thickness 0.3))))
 (gr_line (start 145.05 145.95) (end 145.05 144.8) (angle 90) (layer Edge.Cuts) (width 0.15))
 (gr_line (start 116.8 141) (end 119.25 141) (angle 90) (layer Edge.Cuts) (width 0.15))
 (gr_line (start 116.8 141) (end 118.1 141) (angle 90) (layer Edge.Cuts) (width 0.15))
 (gr_line (start 111.9 145.45) (end 111.95 145.45) (angle 90) (layer Edge.Cuts) (width 0.15))
 (gr_line (start 111.9 146) (end 111.9 145.45) (angle 90) (layer Edge.Cuts) (width 0.15))
 (gr_line (start 138 183.1) (end 118.15 183.1) (angle 90) (layer Edge.Cuts) (width 0.15))
 (gr_line (start 145 145.3) (end 145 144.8) (angle 90) (layer Edge.Cuts) (width 0.15))
 (gr_line (start 111.95 145.7) (end 111.95 175.7) (angle 90) (layer Edge.Cuts) (width 0.15))
 (gr_line (start 145 144.95) (end 145 177.25) (angle 90) (layer Edge.Cuts) (width 0.15))
 (gr_arc (start 138.55 176.65) (end 145 177.2) (angle 90) (layer Edge.Cuts) (width 0.15))
 (gr_line (start 111.9 175.65) (end 111.9 176.65) (angle 90) (layer Edge.Cuts) (width 0.15))
 (gr_arc (start 118.4 176.6) (end 118.1 183.1) (angle 90) (layer Edge.Cuts) (width 0.15))
 (gr_line (start 117.6 141.05) (end 140 141.05) (angle 90) (layer Edge.Cuts) (width 0.15))
 (gr_arc (start 140.65 145.45) (end 139.95 141.05) (angle 90) (layer Edge.Cuts) (width 0.15))
 (gr_arc (start 117.05 146.15) (end 111.9 145.55) (angle 90) (layer Edge.Cuts) (width 0.15))
 (segment (start 116.25 176.25) (end 115.7986 175.7986) (width 0.6) (layer F.Cu) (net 3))
 (segment (start 115.7986 175.7986) (end 115.7986 171.196) (width 0.6) (layer F.Cu) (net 3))
 (segment (start 117.5 176.25) (end 116.25 176.25) (width 0.6) (layer F.Cu) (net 3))
 (segment (start 119.48 178.23) (end 117.5 176.25) (width 0.6) (layer F.Cu) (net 3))
 (segment (start 115.7986 171.196) (end 115.7986 168.656) (width 2.54) (layer F.Cu) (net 3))
 (segment (start 115.7986 166.116) (end 115.7986 168.656) (width 2.54) (layer F.Cu) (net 3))
 (segment (start 115.7986 163.576) (end 115.7986 166.116) (width 2.54) (layer F.Cu) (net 3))
 (segment (start 115.7986 161.036) (end 115.7986 163.576) (width 2.54) (layer F.Cu) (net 3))
 (segment (start 115.7986 158.496) (end 115.7986 161.036) (width 2.54) (layer F.Cu) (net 3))
 (segment (start 115.7986 155.956) (end 115.7986 158.496) (width 2.54) (layer F.Cu) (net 3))
 (segment (start 115.7986 153.416) (end 115.7986 155.956) (width 2.54) (layer F.Cu) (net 3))
 (segment (start 115.7986 171.196) (end 115.7986 153.416) (width 2.54) (layer F.Cu) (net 3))
 (segment (start 127.23 178.23) (end 119.48 178.23) (width 0.6) (layer F.Cu) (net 3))
 (segment (start 127.23 180.77) (end 126.027919 180.77) (width 0.6) (layer B.Cu) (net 4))
 (segment (start 140 176.25) (end 141.224 175.026) (width 0.6) (layer B.Cu) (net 4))
 (segment (start 141.224 175.026) (end 141.224 171.196) (width 0.6) (layer B.Cu) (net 4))
 (segment (start 125 176.25) (end 140 176.25) (width 0.6) (layer B.Cu) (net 4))
 (segment (start 124.25 177) (end 125 176.25) (width 0.6) (layer B.Cu) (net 4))
 (segment (start 124.25 179) (end 124.25 177) (width 0.6) (layer B.Cu) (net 4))
 (segment (start 125.75 180.5) (end 124.25 179) (width 0.6) (layer B.Cu) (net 4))
 (segment (start 125.757919 180.5) (end 125.75 180.5) (width 0.6) (layer B.Cu) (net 4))
 (segment (start 126.027919 180.77) (end 125.757919 180.5) (width 0.6) (layer B.Cu) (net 4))
 (segment (start 141.224 155.956) (end 141.224 153.416) (width 2.54) (layer F.Cu) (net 4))
 (segment (start 141.224 158.496) (end 141.224 155.956) (width 2.54) (layer F.Cu) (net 4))
 (segment (start 141.224 161.036) (end 141.224 158.496) (width 2.54) (layer F.Cu) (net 4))
 (segment (start 141.224 163.576) (end 141.224 161.036) (width 2.54) (layer F.Cu) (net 4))
 (segment (start 141.224 163.576) (end 141.224 166.116) (width 2.54) (layer F.Cu) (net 4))
 (segment (start 141.224 168.656) (end 141.224 166.116) (width 2.54) (layer F.Cu) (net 4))
 (segment (start 141.224 171.196) (end 141.224 168.656) (width 2.54) (layer F.Cu) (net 4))
 (segment (start 143.5 151.75) (end 142.626 150.876) (width 0.6) (layer B.Cu) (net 1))
 (segment (start 142.626 150.876) (end 138.684 150.876) (width 0.6) (layer B.Cu) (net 1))
 (segment (start 143.5 174.25) (end 143.5 151.75) (width 0.6) (layer B.Cu) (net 1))
 (segment (start 140.5 177.25) (end 143.5 174.25) (width 0.6) (layer B.Cu) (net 1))
 (segment (start 134.75 177.25) (end 140.5 177.25) (width 0.6) (layer B.Cu) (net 1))
 (segment (start 133.77 178.23) (end 134.75 177.25) (width 0.6) (layer B.Cu) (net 1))
 (segment (start 120.904 150.876) (end 118.364 150.876) (width 2.54) (layer F.Cu) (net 1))
 (segment (start 123.444 150.876) (end 120.904 150.876) (width 2.54) (layer F.Cu) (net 1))
 (segment (start 125.984 150.876) (end 123.444 150.876) (width 2.54) (layer F.Cu) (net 1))
 (segment (start 128.524 150.876) (end 125.984 150.876) (width 2.54) (layer F.Cu) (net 1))
 (segment (start 131.064 150.876) (end 128.524 150.876) (width 2.54) (layer F.Cu) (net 1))
 (segment (start 133.604 150.876) (end 131.064 150.876) (width 2.54) (layer F.Cu) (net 1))
 (segment (start 136.144 150.876) (end 133.604 150.876) (width 2.54) (layer F.Cu) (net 1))
 (segment (start 138.684 150.876) (end 136.144 150.876) (width 2.54) (layer F.Cu) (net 1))
 (segment (start 129.77 178.23) (end 133.77 178.23) (width 0.6) (layer B.Cu) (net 1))
 (segment (start 129.77 180.77) (end 133.604 176.936) (width 0.6) (layer F.Cu) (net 2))
 (segment (start 133.604 176.936) (end 133.604 173.736) (width 0.6) (layer F.Cu) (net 2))
 (segment (start 136.144 173.736) (end 138.684 173.736) (width 2.54) (layer F.Cu) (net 2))
 (segment (start 133.604 173.736) (end 136.144 173.736) (width 2.54) (layer F.Cu) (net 2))
 (segment (start 133.604 173.736) (end 131.064 173.736) (width 2.54) (layer F.Cu) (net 2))
 (segment (start 128.524 173.736) (end 131.064 173.736) (width 2.54) (layer F.Cu) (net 2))
 (segment (start 125.984 173.736) (end 128.524 173.736) (width 2.54) (layer F.Cu) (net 2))
 (segment (start 123.444 173.736) (end 125.984 173.736) (width 2.54) (layer F.Cu) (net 2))
 (segment (start 120.904 173.736) (end 123.444 173.736) (width 2.54) (layer F.Cu) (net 2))
 (segment (start 118.364 173.736) (end 120.904 173.736) (width 2.54) (layer F.Cu) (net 2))
 (segment (start 118.364 173.736) (end 138.684 173.736) (width 2.54) (layer F.Cu) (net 2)))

